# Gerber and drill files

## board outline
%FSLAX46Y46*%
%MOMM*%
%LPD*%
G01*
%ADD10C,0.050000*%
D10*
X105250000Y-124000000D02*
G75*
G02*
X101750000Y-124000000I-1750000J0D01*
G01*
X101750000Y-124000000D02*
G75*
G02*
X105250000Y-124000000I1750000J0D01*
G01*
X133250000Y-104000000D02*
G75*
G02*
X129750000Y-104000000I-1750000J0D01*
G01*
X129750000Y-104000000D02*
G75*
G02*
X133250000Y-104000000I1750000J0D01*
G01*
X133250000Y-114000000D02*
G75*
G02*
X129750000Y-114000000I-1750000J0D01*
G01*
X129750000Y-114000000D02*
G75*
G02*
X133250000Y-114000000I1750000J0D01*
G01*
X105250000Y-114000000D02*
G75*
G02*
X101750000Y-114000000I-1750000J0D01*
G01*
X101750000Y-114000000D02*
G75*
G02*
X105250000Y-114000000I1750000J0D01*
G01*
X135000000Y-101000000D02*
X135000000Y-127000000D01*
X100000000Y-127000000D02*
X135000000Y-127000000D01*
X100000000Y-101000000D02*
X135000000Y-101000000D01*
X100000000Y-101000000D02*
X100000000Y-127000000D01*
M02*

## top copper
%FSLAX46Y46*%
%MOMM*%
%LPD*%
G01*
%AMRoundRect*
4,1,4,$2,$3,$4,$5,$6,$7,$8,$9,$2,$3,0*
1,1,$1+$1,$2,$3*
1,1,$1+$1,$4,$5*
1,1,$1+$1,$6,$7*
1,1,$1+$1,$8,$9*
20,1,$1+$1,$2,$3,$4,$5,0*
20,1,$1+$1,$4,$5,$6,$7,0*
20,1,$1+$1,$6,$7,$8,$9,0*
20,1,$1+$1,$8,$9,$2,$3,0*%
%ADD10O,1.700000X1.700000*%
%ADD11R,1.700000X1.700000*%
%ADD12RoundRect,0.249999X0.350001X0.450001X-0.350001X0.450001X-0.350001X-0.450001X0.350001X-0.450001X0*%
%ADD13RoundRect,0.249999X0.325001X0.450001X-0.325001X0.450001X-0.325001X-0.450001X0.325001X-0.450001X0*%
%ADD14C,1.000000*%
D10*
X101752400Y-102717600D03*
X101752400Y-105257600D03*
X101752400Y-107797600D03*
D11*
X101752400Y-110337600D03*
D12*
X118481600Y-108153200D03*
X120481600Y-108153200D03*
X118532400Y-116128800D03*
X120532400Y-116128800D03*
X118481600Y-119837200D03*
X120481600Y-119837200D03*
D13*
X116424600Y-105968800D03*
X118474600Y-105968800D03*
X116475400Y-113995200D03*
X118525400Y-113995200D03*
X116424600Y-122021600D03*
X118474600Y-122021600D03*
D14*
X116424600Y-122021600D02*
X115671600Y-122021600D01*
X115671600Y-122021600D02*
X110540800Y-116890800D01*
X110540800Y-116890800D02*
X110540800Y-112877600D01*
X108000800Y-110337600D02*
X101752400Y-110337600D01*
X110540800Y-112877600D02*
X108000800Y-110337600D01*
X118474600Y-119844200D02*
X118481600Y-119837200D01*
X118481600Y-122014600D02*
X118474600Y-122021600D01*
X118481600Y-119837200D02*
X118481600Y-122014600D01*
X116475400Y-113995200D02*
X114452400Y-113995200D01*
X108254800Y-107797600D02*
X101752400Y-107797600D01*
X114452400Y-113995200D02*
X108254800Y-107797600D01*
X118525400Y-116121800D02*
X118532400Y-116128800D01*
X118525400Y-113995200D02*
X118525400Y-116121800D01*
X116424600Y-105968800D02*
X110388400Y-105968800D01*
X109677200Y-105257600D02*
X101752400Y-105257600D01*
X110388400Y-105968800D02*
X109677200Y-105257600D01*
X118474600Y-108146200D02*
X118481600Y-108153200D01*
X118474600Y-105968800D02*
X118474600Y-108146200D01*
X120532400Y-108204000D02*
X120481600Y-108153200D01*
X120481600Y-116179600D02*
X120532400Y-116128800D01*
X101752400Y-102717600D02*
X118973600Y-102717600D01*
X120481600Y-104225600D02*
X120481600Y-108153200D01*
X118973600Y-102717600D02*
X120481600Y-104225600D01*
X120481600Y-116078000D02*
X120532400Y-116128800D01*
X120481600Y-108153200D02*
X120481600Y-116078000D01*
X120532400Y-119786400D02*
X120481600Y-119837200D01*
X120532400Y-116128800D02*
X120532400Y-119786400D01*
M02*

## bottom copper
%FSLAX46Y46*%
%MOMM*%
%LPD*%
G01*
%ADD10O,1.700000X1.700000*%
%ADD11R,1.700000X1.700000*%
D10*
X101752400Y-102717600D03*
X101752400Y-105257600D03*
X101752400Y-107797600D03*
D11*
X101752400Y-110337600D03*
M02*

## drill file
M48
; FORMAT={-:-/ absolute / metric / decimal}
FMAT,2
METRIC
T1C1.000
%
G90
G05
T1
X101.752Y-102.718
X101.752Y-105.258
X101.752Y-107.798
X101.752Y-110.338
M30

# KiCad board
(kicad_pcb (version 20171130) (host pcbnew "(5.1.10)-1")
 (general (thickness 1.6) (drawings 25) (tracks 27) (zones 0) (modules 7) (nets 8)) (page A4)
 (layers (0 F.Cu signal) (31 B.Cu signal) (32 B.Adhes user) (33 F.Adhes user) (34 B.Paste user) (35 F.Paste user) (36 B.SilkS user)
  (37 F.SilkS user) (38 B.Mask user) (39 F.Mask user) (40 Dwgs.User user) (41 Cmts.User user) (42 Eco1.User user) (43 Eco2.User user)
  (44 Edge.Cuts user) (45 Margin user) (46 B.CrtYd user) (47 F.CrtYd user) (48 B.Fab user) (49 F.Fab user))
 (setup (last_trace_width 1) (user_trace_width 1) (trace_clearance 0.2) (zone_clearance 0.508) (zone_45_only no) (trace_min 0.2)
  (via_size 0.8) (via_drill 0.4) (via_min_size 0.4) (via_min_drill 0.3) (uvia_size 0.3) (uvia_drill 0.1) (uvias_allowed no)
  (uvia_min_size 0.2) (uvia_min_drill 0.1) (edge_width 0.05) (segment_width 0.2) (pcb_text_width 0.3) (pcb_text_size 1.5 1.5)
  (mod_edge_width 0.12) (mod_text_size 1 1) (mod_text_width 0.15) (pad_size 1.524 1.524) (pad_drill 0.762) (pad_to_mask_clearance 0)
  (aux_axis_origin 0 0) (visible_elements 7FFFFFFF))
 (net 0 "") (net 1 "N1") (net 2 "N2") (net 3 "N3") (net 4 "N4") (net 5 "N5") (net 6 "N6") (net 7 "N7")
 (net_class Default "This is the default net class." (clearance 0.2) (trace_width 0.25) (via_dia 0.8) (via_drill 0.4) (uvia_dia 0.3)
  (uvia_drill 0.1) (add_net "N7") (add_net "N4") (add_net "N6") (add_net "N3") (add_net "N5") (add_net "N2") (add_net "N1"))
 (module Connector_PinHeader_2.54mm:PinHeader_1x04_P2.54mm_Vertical (layer F.Cu) (at 101.7524 110.3376 180)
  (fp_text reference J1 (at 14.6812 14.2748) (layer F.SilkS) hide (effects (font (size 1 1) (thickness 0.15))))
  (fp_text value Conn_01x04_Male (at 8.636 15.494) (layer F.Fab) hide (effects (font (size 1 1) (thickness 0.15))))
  (pad 4 thru_hole oval (at 0 7.62 180) (size 1.7 1.7) (drill 1) (layers *.Cu *.Mask) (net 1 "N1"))
  (pad 3 thru_hole oval (at 0 5.08 180) (size 1.7 1.7) (drill 1) (layers *.Cu *.Mask) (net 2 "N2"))
  (pad 2 thru_hole oval (at 0 2.54 180) (size 1.7 1.7) (drill 1) (layers *.Cu *.Mask) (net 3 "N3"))
  (pad 1 thru_hole rect (at 0 0 180) (size 1.7 1.7) (drill 1) (layers *.Cu *.Mask) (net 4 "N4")))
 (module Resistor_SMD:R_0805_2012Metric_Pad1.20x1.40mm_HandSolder (layer F.Cu) (at 119.4816 108.1532 180)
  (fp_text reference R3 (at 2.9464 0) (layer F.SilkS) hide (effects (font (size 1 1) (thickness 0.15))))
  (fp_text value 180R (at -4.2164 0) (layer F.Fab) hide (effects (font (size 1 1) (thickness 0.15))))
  (pad 2 smd roundrect (at 1 0 180) (size 1.2 1.4) (layers F.Cu F.Paste F.Mask) (roundrect_rratio 0.2083325) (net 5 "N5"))
  (pad 1 smd roundrect (at -1 0 180) (size 1.2 1.4) (layers F.Cu F.Paste F.Mask) (roundrect_rratio 0.2083325) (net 1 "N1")))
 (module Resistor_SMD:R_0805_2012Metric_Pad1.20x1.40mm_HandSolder (layer F.Cu) (at 119.5324 116.1288 180)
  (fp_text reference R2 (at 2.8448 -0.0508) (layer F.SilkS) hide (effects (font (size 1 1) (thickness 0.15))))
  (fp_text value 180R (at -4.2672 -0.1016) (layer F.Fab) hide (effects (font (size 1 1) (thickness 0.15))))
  (pad 2 smd roundrect (at 1 0 180) (size 1.2 1.4) (layers F.Cu F.Paste F.Mask) (roundrect_rratio 0.2083325) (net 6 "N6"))
  (pad 1 smd roundrect (at -1 0 180) (size 1.2 1.4) (layers F.Cu F.Paste F.Mask) (roundrect_rratio 0.2083325) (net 1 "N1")))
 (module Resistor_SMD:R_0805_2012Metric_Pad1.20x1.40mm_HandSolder (layer F.Cu) (at 119.4816 119.8372 180)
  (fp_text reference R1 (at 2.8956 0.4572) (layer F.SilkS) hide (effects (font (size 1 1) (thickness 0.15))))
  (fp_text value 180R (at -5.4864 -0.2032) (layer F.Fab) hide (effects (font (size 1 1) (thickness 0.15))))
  (pad 2 smd roundrect (at 1 0 180) (size 1.2 1.4) (layers F.Cu F.Paste F.Mask) (roundrect_rratio 0.2083325) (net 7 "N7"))
  (pad 1 smd roundrect (at -1 0 180) (size 1.2 1.4) (layers F.Cu F.Paste F.Mask) (roundrect_rratio 0.2083325) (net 1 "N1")))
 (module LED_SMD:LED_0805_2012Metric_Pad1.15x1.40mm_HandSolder (layer F.Cu) (at 117.4496 105.9688 180)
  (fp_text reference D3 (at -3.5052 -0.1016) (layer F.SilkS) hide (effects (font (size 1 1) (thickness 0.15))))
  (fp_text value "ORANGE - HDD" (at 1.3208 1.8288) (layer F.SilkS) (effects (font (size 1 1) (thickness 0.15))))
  (pad 2 smd roundrect (at 1.025 0 180) (size 1.15 1.4) (layers F.Cu F.Paste F.Mask) (roundrect_rratio 0.2173904347826087) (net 2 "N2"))
  (pad 1 smd roundrect (at -1.025 0 180) (size 1.15 1.4) (layers F.Cu F.Paste F.Mask) (roundrect_rratio 0.2173904347826087) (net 5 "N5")))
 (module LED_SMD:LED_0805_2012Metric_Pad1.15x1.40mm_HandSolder (layer F.Cu) (at 117.5004 113.9952 180)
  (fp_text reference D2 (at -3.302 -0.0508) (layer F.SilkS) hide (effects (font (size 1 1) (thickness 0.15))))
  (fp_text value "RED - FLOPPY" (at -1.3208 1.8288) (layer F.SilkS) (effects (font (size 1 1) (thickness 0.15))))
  (pad 2 smd roundrect (at 1.025 0 180) (size 1.15 1.4) (layers F.Cu F.Paste F.Mask) (roundrect_rratio 0.2173904347826087) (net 3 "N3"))
  (pad 1 smd roundrect (at -1.025 0 180) (size 1.15 1.4) (layers F.Cu F.Paste F.Mask) (roundrect_rratio 0.2173904347826087) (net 6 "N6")))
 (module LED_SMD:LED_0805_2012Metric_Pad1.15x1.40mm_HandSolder (layer F.Cu) (at 117.4496 122.0216 180)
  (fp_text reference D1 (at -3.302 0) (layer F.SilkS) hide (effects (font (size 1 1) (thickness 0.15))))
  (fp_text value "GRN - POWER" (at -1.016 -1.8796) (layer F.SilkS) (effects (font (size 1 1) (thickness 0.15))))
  (pad 2 smd roundrect (at 1.025 0 180) (size 1.15 1.4) (layers F.Cu F.Paste F.Mask) (roundrect_rratio 0.2173904347826087) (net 4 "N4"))
  (pad 1 smd roundrect (at -1.025 0 180) (size 1.15 1.4) (layers F.Cu F.Paste F.Mask) (roundrect_rratio 0.2173904347826087) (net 7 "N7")))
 (gr_circle (center 103.5 124) (end 105.25 124) (layer Edge.Cuts) (width 0.05))
 (gr_circle (center 131.5 104) (end 133.25 104) (layer Edge.Cuts) (width 0.05))
 (gr_circle (center 131.5 114) (end 133.25 114) (layer Edge.Cuts) (width 0.05))
 (gr_circle (center 103.5 114) (end 105.25 114) (layer Edge.Cuts) (width 0.05))
 (gr_line (start 135 101) (end 135 127) (layer Edge.Cuts) (width 0.05))
 (gr_line (start 100 127) (end 135 127) (layer Edge.Cuts) (width 0.05))
 (gr_line (start 100 101) (end 135 101) (layer Edge.Cuts) (width 0.05))
 (gr_line (start 100 101) (end 100 127) (layer Edge.Cuts) (width 0.05))
 (segment (start 116.4246 122.0216) (end 115.6716 122.0216) (width 1) (layer F.Cu) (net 4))
 (segment (start 115.6716 122.0216) (end 110.5408 116.8908) (width 1) (layer F.Cu) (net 4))
 (segment (start 110.5408 116.8908) (end 110.5408 112.8776) (width 1) (layer F.Cu) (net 4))
 (segment (start 108.0008 110.3376) (end 101.7524 110.3376) (width 1) (layer F.Cu) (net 4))
 (segment (start 110.5408 112.8776) (end 108.0008 110.3376) (width 1) (layer F.Cu) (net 4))
 (segment (start 118.4746 119.8442) (end 118.4816 119.8372) (width 1) (layer F.Cu) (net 7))
 (segment (start 118.4816 122.0146) (end 118.4746 122.0216) (width 1) (layer F.Cu) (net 7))
 (segment (start 118.4816 119.8372) (end 118.4816 122.0146) (width 1) (layer F.Cu) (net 7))
 (segment (start 116.4754 113.9952) (end 114.4524 113.9952) (width 1) (layer F.Cu) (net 3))
 (segment (start 108.2548 107.7976) (end 101.7524 107.7976) (width 1) (layer F.Cu) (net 3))
 (segment (start 114.4524 113.9952) (end 108.2548 107.7976) (width 1) (layer F.Cu) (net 3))
 (segment (start 118.5254 116.1218) (end 118.5324 116.1288) (width 1) (layer F.Cu) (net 6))
 (segment (start 118.5254 113.9952) (end 118.5254 116.1218) (width 1) (layer F.Cu) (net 6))
 (segment (start 116.4246 105.9688) (end 110.3884 105.9688) (width 1) (layer F.Cu) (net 2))
 (segment (start 109.6772 105.2576) (end 101.7524 105.2576) (width 1) (layer F.Cu) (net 2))
 (segment (start 110.3884 105.9688) (end 109.6772 105.2576) (width 1) (layer F.Cu) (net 2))
 (segment (start 118.4746 108.1462) (end 118.4816 108.1532) (width 1) (layer F.Cu) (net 5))
 (segment (start 118.4746 105.9688) (end 118.4746 108.1462) (width 1) (layer F.Cu) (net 5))
 (segment (start 120.5324 108.204) (end 120.4816 108.1532) (width 1) (layer F.Cu) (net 1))
 (segment (start 120.4816 116.1796) (end 120.5324 116.1288) (width 1) (layer F.Cu) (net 1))
 (segment (start 101.7524 102.7176) (end 118.9736 102.7176) (width 1) (layer F.Cu) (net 1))
 (segment (start 120.4816 104.2256) (end 120.4816 108.1532) (width 1) (layer F.Cu) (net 1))
 (segment (start 118.9736 102.7176) (end 120.4816 104.2256) (width 1) (layer F.Cu) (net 1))
 (segment (start 120.4816 116.078) (end 120.5324 116.1288) (width 1) (layer F.Cu) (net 1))
 (segment (start 120.4816 108.1532) (end 120.4816 116.078) (width 1) (layer F.Cu) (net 1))
 (segment (start 120.5324 119.7864) (end 120.4816 119.8372) (width 1) (layer F.Cu) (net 1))
 (segment (start 120.5324 116.1288) (end 120.5324 119.7864) (width 1) (layer F.Cu) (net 1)))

